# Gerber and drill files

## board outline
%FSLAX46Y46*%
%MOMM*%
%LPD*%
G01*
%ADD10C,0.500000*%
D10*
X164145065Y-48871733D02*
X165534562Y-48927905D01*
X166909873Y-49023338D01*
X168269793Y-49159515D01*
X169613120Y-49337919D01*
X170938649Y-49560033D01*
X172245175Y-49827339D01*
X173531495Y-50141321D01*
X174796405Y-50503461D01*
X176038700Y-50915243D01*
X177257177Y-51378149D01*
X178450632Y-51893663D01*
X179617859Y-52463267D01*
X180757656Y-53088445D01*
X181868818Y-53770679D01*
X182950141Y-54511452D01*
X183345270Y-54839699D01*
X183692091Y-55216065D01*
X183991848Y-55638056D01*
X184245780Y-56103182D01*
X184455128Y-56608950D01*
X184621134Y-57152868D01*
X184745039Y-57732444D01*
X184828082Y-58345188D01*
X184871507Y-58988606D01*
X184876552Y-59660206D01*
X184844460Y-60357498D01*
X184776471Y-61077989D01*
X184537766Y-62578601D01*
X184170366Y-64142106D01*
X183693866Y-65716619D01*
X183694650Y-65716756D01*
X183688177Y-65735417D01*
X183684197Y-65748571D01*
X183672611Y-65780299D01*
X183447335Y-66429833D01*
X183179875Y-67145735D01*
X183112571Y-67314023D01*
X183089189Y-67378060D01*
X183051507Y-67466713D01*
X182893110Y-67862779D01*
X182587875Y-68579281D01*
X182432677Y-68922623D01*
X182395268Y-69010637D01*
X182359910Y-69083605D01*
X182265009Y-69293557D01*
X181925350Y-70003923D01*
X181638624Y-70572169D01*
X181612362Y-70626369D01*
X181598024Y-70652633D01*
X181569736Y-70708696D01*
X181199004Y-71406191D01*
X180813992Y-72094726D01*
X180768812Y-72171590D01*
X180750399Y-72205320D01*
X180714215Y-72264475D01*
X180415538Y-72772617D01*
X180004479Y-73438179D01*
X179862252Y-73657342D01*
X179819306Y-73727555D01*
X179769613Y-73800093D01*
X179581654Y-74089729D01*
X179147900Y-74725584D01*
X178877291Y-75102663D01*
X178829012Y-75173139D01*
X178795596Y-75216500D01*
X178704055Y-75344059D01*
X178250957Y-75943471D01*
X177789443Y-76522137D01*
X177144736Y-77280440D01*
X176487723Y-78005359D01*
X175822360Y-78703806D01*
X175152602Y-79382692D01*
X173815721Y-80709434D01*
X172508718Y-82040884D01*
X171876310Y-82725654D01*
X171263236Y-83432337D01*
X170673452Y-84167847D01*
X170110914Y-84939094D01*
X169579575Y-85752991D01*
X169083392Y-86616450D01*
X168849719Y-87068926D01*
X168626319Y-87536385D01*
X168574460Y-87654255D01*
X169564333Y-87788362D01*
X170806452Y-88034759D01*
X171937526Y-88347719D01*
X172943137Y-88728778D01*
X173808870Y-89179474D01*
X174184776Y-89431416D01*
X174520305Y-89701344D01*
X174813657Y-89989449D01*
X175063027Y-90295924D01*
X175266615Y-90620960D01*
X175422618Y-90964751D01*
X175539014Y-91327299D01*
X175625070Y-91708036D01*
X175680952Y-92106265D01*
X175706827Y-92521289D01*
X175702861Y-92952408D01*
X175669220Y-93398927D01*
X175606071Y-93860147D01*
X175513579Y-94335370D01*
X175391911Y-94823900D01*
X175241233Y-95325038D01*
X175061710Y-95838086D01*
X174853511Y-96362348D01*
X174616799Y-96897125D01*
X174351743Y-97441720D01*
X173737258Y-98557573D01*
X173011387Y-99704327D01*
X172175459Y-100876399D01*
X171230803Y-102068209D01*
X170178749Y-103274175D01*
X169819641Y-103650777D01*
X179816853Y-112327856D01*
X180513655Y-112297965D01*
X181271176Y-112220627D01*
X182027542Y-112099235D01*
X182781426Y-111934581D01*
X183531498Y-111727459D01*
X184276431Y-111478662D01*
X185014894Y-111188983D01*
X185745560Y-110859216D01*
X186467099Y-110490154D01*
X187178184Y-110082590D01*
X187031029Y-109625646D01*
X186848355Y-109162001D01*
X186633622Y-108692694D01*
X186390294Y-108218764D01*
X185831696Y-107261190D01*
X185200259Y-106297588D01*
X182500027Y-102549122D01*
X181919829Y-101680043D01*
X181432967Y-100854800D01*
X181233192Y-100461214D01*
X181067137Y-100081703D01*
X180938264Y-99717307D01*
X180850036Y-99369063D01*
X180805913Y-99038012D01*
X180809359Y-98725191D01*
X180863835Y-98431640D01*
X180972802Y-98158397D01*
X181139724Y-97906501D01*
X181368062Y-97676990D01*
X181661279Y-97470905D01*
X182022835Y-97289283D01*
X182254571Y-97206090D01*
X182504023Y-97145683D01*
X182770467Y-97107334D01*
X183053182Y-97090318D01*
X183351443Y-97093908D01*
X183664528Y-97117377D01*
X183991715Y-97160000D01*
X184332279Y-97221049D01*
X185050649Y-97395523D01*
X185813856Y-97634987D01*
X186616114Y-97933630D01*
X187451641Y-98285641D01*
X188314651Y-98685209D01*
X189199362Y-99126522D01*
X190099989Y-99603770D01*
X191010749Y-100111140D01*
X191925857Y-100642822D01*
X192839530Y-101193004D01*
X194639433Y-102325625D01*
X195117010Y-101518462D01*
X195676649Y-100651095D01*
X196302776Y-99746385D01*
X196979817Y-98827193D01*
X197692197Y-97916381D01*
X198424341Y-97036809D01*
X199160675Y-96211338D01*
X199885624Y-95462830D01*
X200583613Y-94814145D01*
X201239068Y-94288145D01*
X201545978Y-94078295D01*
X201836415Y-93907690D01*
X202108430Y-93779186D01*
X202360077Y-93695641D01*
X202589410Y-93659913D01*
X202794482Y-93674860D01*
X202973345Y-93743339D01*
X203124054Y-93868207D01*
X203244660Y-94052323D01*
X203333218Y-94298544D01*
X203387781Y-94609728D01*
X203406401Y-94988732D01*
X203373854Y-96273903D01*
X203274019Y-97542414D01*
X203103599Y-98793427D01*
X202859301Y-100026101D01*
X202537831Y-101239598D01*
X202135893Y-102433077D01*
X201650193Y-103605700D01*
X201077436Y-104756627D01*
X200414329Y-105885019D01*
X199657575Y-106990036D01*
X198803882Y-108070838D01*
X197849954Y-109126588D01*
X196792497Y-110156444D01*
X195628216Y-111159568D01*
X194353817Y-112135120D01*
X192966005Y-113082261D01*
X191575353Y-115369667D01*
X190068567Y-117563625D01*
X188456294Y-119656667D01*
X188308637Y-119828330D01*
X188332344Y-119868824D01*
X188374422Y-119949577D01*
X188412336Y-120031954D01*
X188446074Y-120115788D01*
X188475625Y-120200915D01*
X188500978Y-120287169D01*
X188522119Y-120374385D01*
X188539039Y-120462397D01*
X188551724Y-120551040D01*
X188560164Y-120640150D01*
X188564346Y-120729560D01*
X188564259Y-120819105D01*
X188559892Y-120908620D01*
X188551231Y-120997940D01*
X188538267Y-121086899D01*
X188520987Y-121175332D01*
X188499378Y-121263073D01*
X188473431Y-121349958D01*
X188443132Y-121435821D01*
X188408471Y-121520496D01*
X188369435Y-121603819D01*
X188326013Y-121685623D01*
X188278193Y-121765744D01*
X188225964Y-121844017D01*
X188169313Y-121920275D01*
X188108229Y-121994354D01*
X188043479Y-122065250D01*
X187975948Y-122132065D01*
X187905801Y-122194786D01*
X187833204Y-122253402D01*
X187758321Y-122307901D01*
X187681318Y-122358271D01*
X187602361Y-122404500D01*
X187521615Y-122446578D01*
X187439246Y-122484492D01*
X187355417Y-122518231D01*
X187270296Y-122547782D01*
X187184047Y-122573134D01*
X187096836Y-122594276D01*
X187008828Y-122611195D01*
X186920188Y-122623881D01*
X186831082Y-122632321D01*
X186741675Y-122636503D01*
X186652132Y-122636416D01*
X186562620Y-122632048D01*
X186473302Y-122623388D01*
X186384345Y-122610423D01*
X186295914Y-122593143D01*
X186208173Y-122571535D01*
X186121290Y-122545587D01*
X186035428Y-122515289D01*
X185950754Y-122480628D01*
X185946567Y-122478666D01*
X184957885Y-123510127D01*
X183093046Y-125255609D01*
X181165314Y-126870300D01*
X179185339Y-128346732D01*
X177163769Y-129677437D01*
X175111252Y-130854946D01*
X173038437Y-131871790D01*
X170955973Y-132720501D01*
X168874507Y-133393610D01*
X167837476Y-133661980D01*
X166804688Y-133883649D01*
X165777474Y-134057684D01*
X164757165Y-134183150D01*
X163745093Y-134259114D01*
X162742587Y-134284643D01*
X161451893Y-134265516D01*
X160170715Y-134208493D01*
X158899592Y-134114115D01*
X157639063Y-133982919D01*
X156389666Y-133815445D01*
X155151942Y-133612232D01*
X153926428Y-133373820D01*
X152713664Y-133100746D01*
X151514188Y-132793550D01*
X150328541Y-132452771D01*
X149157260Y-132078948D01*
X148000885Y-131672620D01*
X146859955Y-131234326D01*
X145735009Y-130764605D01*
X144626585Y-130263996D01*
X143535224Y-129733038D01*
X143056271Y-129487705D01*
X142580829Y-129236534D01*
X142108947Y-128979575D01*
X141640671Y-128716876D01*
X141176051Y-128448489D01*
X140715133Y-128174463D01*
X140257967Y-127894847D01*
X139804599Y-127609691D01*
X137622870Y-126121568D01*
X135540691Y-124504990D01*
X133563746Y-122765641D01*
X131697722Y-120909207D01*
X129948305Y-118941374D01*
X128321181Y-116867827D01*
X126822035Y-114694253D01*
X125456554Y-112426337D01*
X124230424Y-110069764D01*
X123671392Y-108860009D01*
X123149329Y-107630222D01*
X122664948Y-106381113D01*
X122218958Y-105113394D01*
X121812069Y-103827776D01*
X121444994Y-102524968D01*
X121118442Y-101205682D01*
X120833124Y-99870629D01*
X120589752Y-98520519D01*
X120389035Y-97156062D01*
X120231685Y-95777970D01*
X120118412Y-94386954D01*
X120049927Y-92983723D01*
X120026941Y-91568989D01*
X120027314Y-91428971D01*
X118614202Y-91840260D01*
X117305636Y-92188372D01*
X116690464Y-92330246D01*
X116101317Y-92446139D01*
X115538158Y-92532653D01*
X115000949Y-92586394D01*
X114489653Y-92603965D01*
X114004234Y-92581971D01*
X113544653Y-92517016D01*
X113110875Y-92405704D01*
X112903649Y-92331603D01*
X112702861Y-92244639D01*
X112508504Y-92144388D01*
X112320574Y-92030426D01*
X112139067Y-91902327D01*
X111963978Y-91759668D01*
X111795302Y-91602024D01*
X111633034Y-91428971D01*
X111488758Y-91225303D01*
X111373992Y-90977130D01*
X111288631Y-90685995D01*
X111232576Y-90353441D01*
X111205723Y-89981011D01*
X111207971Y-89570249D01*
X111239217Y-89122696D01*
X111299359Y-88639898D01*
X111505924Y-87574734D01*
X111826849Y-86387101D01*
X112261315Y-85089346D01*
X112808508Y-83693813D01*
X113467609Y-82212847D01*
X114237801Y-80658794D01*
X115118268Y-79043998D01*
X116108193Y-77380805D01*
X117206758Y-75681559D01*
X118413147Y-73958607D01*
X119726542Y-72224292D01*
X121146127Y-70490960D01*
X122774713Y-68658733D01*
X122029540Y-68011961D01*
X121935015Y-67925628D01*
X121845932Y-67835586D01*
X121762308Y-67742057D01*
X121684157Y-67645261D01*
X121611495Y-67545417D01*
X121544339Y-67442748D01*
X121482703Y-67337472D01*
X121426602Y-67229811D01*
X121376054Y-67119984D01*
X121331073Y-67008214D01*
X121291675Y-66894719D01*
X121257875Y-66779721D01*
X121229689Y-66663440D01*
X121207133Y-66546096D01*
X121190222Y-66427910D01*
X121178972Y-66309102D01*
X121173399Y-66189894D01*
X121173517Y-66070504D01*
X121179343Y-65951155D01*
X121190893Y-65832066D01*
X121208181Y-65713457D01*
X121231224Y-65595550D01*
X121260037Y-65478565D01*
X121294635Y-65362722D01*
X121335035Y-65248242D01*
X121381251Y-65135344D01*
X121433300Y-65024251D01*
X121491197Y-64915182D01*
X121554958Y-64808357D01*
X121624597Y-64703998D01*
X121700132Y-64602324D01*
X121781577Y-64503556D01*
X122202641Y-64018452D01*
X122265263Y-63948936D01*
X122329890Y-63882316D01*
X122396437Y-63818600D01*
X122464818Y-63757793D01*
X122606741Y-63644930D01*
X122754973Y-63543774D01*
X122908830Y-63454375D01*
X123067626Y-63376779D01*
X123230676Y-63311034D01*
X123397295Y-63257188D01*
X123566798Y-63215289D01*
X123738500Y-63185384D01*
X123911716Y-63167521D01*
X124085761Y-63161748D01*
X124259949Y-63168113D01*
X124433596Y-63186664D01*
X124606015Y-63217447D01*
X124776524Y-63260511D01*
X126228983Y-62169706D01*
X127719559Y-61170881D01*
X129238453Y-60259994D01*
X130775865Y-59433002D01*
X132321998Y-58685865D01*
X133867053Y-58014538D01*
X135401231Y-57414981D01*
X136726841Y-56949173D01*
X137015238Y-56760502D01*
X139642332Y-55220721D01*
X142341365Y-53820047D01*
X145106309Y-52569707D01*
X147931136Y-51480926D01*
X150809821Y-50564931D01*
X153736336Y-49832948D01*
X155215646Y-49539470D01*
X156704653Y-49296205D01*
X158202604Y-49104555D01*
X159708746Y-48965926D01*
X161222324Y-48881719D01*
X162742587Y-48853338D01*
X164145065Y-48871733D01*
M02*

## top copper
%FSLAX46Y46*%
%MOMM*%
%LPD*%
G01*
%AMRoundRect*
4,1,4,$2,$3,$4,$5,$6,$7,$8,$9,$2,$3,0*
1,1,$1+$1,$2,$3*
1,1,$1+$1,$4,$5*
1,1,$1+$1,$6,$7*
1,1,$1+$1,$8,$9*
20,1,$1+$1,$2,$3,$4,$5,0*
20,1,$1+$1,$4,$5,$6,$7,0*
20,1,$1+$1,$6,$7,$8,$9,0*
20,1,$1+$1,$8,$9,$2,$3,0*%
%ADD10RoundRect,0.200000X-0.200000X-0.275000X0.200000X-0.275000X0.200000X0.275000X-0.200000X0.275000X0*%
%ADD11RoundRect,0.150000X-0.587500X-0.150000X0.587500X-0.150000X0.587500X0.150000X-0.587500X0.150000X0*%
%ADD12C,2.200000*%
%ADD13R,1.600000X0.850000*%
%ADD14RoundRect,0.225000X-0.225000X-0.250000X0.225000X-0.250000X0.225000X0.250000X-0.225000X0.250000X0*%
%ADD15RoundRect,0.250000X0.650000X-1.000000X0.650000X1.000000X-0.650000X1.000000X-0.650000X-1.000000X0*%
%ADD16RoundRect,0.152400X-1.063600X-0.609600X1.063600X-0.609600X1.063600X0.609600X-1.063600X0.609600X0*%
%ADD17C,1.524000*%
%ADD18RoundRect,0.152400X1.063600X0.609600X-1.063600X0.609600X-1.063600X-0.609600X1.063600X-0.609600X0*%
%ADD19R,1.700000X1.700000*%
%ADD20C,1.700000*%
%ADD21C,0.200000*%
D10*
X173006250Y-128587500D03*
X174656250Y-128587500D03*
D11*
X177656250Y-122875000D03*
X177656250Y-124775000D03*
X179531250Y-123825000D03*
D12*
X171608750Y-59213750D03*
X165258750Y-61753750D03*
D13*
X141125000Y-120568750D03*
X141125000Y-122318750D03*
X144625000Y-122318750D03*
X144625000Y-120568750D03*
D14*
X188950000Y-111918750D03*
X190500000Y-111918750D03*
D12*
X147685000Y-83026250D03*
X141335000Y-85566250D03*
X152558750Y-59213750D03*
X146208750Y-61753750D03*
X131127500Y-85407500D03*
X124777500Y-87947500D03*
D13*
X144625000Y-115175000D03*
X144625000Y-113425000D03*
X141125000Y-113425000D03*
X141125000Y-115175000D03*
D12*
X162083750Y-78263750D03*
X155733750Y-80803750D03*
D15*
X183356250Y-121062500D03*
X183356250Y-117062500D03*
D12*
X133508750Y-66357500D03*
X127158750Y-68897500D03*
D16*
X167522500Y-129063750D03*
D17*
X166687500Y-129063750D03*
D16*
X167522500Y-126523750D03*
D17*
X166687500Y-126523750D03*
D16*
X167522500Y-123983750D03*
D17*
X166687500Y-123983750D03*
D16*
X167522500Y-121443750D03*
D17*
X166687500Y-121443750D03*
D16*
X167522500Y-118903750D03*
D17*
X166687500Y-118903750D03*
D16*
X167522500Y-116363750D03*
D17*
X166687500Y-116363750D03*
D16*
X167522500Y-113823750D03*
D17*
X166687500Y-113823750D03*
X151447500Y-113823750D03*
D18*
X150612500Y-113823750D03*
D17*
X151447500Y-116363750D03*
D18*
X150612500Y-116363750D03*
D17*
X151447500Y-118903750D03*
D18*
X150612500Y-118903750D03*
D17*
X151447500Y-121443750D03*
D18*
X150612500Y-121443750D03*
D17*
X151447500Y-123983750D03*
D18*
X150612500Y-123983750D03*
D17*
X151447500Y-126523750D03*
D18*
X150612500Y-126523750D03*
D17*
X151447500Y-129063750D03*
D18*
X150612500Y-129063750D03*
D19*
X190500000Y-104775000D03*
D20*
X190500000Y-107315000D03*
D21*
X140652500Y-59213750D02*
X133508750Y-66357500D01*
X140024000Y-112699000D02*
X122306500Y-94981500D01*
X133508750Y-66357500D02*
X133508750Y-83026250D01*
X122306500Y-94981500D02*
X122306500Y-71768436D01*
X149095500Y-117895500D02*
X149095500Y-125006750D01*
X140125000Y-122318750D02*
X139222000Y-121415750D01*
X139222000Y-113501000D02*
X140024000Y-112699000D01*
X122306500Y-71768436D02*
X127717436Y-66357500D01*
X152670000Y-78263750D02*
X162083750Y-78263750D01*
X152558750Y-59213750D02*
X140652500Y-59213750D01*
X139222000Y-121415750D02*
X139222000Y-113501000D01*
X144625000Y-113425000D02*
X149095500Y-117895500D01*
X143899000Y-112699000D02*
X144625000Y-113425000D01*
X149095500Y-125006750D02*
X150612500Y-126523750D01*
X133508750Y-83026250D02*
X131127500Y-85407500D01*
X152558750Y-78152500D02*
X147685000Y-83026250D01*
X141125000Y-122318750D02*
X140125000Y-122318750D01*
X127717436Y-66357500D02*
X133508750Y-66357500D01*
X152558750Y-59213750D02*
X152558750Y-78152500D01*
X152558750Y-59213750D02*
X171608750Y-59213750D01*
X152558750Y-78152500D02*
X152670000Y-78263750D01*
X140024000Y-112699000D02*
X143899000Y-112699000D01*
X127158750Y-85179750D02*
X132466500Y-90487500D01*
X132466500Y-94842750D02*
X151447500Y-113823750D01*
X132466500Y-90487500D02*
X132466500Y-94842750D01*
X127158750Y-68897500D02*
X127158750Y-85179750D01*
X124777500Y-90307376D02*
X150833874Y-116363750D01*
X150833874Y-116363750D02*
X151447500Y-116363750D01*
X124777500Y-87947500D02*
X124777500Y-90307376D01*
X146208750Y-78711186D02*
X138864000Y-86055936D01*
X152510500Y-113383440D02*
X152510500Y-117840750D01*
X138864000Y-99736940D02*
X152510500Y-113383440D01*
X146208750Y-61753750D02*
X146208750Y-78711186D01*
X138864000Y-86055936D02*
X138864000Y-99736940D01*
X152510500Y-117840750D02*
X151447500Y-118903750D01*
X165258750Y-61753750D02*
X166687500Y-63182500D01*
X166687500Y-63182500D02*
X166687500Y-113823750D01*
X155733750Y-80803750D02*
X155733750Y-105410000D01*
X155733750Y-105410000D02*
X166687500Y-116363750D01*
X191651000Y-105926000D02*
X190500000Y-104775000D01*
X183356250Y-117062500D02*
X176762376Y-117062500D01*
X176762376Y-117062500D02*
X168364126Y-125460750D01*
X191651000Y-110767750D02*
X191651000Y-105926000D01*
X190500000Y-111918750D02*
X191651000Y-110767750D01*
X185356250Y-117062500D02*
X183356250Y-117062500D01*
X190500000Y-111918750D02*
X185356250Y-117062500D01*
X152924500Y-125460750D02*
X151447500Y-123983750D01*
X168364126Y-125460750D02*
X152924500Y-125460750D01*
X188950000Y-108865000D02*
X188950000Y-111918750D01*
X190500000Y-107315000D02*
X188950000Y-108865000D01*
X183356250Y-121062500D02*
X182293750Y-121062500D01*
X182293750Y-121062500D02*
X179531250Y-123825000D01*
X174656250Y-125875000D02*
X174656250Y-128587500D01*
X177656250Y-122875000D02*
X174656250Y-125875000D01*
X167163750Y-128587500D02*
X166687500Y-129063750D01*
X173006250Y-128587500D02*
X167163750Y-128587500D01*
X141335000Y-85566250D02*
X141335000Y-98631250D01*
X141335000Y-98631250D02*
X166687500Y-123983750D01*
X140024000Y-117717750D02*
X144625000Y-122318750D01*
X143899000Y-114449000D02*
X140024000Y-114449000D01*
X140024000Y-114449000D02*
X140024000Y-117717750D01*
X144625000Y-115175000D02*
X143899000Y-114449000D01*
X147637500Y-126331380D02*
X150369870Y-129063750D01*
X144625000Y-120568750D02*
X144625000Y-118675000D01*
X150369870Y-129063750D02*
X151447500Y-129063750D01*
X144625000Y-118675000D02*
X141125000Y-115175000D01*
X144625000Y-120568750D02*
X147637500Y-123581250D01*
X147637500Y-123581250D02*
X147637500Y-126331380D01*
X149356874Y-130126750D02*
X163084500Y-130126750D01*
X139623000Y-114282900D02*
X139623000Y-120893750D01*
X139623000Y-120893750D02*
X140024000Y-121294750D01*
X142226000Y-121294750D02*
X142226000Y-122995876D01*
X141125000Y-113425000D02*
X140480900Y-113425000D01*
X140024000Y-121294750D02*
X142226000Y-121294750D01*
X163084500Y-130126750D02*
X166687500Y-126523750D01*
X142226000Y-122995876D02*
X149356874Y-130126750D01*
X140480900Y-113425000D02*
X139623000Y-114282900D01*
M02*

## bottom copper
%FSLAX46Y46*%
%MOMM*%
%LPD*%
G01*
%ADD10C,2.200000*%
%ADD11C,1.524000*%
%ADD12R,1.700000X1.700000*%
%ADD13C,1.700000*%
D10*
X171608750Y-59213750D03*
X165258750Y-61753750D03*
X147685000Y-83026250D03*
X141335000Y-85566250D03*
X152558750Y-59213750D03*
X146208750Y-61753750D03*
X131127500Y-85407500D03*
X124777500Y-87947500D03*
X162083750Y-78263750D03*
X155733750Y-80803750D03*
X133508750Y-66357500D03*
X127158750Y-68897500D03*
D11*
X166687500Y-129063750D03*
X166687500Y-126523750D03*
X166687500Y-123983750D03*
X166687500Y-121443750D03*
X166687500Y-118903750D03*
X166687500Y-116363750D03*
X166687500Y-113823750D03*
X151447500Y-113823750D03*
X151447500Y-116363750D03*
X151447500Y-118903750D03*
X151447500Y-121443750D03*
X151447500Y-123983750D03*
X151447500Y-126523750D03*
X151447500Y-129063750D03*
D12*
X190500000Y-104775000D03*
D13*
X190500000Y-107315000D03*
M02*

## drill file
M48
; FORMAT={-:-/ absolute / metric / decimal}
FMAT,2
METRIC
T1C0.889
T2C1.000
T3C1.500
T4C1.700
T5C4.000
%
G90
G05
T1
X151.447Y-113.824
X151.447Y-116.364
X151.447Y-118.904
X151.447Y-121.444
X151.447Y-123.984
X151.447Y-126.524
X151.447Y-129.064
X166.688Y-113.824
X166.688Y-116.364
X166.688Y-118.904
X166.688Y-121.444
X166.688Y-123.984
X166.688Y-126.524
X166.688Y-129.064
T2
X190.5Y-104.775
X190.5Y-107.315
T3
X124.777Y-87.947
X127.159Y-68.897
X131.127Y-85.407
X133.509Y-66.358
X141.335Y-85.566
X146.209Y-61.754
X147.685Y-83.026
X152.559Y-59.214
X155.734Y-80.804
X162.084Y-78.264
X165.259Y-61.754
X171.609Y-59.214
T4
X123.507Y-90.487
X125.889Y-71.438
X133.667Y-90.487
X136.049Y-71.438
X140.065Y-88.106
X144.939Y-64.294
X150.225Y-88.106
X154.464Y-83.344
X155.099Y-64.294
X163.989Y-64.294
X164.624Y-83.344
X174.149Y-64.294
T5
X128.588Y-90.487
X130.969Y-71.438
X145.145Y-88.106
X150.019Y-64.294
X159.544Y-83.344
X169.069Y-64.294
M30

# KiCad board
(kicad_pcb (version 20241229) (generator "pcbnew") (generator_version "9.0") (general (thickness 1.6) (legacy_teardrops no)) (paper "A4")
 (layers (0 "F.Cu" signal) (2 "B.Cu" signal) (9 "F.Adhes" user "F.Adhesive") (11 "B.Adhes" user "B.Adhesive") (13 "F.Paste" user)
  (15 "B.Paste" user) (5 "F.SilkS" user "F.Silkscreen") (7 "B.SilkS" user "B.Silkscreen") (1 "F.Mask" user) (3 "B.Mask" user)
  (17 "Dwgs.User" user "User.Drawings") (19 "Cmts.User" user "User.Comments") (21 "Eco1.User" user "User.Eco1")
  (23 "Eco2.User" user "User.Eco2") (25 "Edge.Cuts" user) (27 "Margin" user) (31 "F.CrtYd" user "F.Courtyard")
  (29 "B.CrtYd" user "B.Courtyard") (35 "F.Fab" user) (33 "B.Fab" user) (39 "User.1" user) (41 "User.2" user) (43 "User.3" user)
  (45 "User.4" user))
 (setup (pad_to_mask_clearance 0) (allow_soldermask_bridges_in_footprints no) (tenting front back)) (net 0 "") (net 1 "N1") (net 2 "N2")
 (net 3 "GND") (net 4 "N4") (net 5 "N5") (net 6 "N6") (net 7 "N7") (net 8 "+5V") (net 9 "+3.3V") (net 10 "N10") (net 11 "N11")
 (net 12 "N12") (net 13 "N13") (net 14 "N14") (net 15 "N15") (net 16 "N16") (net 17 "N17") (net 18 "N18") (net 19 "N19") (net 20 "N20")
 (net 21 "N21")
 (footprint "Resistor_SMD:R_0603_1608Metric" (layer "F.Cu") (at 173.83125 128.5875)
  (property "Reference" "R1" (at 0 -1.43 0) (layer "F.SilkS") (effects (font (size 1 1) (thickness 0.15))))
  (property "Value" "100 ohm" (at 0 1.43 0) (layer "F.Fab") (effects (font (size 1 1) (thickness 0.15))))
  (pad "1" smd roundrect (at -0.825 0) (size 0.8 0.95) (layers "F.Cu" "F.Mask" "F.Paste") (roundrect_rratio 0.25) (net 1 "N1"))
  (pad "2" smd roundrect (at 0.825 0) (size 0.8 0.95) (layers "F.Cu" "F.Mask" "F.Paste") (roundrect_rratio 0.25) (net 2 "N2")))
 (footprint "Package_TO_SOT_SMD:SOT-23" (layer "F.Cu") (at 178.59375 123.825)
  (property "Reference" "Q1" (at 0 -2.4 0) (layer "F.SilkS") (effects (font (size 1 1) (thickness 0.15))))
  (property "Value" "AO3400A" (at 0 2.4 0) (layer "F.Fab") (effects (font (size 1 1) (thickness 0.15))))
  (pad "1" smd roundrect (at -0.9375 -0.95) (size 1.475 0.6) (layers "F.Cu" "F.Mask" "F.Paste") (roundrect_rratio 0.25) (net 2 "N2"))
  (pad "2" smd roundrect (at -0.9375 0.95) (size 1.475 0.6) (layers "F.Cu" "F.Mask" "F.Paste") (roundrect_rratio 0.25) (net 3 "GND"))
  (pad "3" smd roundrect (at 0.9375 0) (size 1.475 0.6) (layers "F.Cu" "F.Mask" "F.Paste") (roundrect_rratio 0.25) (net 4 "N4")))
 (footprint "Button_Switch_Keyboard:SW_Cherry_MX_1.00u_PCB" (layer "F.Cu") (at 171.60875 59.21375)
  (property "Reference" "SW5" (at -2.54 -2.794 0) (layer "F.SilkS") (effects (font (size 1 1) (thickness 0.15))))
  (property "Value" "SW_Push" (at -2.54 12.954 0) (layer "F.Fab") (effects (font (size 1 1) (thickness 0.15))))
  (pad "" np_thru_hole circle (at -7.62 5.08) (size 1.7 1.7) (drill 1.7) (layers "*.Cu" "*.Mask"))
  (pad "" np_thru_hole circle (at -2.54 5.08) (size 4 4) (drill 4) (layers "*.Cu" "*.Mask"))
  (pad "" np_thru_hole circle (at 2.54 5.08) (size 1.7 1.7) (drill 1.7) (layers "*.Cu" "*.Mask"))
  (pad "1" thru_hole circle (at 0 0) (size 2.2 2.2) (drill 1.5) (layers "*.Cu" "*.Mask") (remove_unused_layers no) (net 3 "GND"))
  (pad "2" thru_hole circle (at -6.35 2.54) (size 2.2 2.2) (drill 1.5) (layers "*.Cu" "*.Mask") (remove_unused_layers no) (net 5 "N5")))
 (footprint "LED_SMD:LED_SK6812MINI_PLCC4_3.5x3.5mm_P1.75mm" (layer "F.Cu") (at 142.875 121.44375)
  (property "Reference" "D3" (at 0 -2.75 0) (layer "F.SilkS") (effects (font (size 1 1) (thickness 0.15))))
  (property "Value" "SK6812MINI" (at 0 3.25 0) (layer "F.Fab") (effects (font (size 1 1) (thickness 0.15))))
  (pad "1" smd rect (at -1.75 -0.875) (size 1.6 0.85) (layers "F.Cu" "F.Mask" "F.Paste") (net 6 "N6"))
  (pad "2" smd rect (at -1.75 0.875) (size 1.6 0.85) (layers "F.Cu" "F.Mask" "F.Paste") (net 3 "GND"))
  (pad "3" smd rect (at 1.75 0.875) (size 1.6 0.85) (layers "F.Cu" "F.Mask" "F.Paste") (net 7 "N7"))
  (pad "4" smd rect (at 1.75 -0.875) (size 1.6 0.85) (layers "F.Cu" "F.Mask" "F.Paste") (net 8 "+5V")))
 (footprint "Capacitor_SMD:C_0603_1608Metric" (layer "F.Cu") (at 189.725 111.91875)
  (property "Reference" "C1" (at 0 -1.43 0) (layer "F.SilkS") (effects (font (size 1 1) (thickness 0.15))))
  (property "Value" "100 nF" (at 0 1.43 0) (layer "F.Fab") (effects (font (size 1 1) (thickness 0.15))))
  (pad "1" smd roundrect (at -0.775 0) (size 0.9 0.95) (layers "F.Cu" "F.Mask" "F.Paste") (roundrect_rratio 0.25) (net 4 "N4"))
  (pad "2" smd roundrect (at 0.775 0) (size 0.9 0.95) (layers "F.Cu" "F.Mask" "F.Paste") (roundrect_rratio 0.25) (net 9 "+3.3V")))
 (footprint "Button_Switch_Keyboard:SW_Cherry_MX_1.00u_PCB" (layer "F.Cu") (at 147.685 83.02625)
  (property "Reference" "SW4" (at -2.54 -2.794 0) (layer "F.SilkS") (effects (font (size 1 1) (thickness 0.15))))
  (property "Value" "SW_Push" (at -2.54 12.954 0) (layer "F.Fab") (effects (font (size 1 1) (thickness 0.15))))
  (pad "" np_thru_hole circle (at -7.62 5.08) (size 1.7 1.7) (drill 1.7) (layers "*.Cu" "*.Mask"))
  (pad "" np_thru_hole circle (at -2.54 5.08) (size 4 4) (drill 4) (layers "*.Cu" "*.Mask"))
  (pad "" np_thru_hole circle (at 2.54 5.08) (size 1.7 1.7) (drill 1.7) (layers "*.Cu" "*.Mask"))
  (pad "1" thru_hole circle (at 0 0) (size 2.2 2.2) (drill 1.5) (layers "*.Cu" "*.Mask") (remove_unused_layers no) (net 3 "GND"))
  (pad "2" thru_hole circle (at -6.35 2.54) (size 2.2 2.2) (drill 1.5) (layers "*.Cu" "*.Mask") (remove_unused_layers no) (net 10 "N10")))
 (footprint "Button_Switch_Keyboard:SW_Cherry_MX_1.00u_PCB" (layer "F.Cu") (at 152.55875 59.21375)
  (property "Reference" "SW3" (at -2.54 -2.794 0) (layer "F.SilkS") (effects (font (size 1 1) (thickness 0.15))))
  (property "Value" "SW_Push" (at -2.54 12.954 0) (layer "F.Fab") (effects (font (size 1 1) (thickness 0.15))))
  (pad "" np_thru_hole circle (at -7.62 5.08) (size 1.7 1.7) (drill 1.7) (layers "*.Cu" "*.Mask"))
  (pad "" np_thru_hole circle (at -2.54 5.08) (size 4 4) (drill 4) (layers "*.Cu" "*.Mask"))
  (pad "" np_thru_hole circle (at 2.54 5.08) (size 1.7 1.7) (drill 1.7) (layers "*.Cu" "*.Mask"))
  (pad "1" thru_hole circle (at 0 0) (size 2.2 2.2) (drill 1.5) (layers "*.Cu" "*.Mask") (remove_unused_layers no) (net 3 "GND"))
  (pad "2" thru_hole circle (at -6.35 2.54) (size 2.2 2.2) (drill 1.5) (layers "*.Cu" "*.Mask") (remove_unused_layers no) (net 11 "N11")))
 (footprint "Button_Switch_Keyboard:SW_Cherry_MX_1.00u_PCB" (layer "F.Cu") (at 131.1275 85.4075)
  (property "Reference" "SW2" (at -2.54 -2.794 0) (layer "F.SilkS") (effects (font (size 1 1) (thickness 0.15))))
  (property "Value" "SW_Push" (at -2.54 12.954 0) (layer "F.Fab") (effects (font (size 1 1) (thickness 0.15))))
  (pad "" np_thru_hole circle (at -7.62 5.08) (size 1.7 1.7) (drill 1.7) (layers "*.Cu" "*.Mask"))
  (pad "" np_thru_hole circle (at -2.54 5.08) (size 4 4) (drill 4) (layers "*.Cu" "*.Mask"))
  (pad "" np_thru_hole circle (at 2.54 5.08) (size 1.7 1.7) (drill 1.7) (layers "*.Cu" "*.Mask"))
  (pad "1" thru_hole circle (at 0 0) (size 2.2 2.2) (drill 1.5) (layers "*.Cu" "*.Mask") (remove_unused_layers no) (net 3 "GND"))
  (pad "2" thru_hole circle (at -6.35 2.54) (size 2.2 2.2) (drill 1.5) (layers "*.Cu" "*.Mask") (remove_unused_layers no) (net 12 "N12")))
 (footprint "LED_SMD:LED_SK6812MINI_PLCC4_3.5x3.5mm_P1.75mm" (layer "F.Cu") (at 142.875 114.3 180)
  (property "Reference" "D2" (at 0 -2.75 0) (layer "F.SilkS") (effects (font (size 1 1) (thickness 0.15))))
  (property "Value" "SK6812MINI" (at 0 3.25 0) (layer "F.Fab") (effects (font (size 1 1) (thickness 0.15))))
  (pad "1" smd rect (at -1.75 -0.875 180) (size 1.6 0.85) (layers "F.Cu" "F.Mask" "F.Paste") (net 7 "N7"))
  (pad "2" smd rect (at -1.75 0.875 180) (size 1.6 0.85) (layers "F.Cu" "F.Mask" "F.Paste") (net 3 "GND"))
  (pad "3" smd rect (at 1.75 0.875 180) (size 1.6 0.85) (layers "F.Cu" "F.Mask" "F.Paste") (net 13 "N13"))
  (pad "4" smd rect (at 1.75 -0.875 180) (size 1.6 0.85) (layers "F.Cu" "F.Mask" "F.Paste") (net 8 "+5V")))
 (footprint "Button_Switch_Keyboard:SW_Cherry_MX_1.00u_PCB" (layer "F.Cu") (at 162.08375 78.26375)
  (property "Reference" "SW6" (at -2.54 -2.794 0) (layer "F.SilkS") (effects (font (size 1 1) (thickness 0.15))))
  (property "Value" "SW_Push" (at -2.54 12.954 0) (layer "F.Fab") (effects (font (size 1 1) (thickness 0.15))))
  (pad "" np_thru_hole circle (at -7.62 5.08) (size 1.7 1.7) (drill 1.7) (layers "*.Cu" "*.Mask"))
  (pad "" np_thru_hole circle (at -2.54 5.08) (size 4 4) (drill 4) (layers "*.Cu" "*.Mask"))
  (pad "" np_thru_hole circle (at 2.54 5.08) (size 1.7 1.7) (drill 1.7) (layers "*.Cu" "*.Mask"))
  (pad "1" thru_hole circle (at 0 0) (size 2.2 2.2) (drill 1.5) (layers "*.Cu" "*.Mask") (remove_unused_layers no) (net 3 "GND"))
  (pad "2" thru_hole circle (at -6.35 2.54) (size 2.2 2.2) (drill 1.5) (layers "*.Cu" "*.Mask") (remove_unused_layers no) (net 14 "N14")))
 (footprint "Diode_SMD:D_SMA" (layer "F.Cu") (at 183.35625 119.0625 90)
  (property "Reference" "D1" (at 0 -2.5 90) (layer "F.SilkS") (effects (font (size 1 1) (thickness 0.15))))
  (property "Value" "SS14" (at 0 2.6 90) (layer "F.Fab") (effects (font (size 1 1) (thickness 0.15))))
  (pad "1" smd roundrect (at -2 0 90) (size 2.5 1.8) (layers "F.Cu" "F.Mask" "F.Paste") (roundrect_rratio 0.1388888889) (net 4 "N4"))
  (pad "2" smd roundrect (at 2 0 90) (size 2.5 1.8) (layers "F.Cu" "F.Mask" "F.Paste") (roundrect_rratio 0.1388888889) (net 9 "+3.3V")))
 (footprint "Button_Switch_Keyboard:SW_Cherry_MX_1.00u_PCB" (layer "F.Cu") (at 133.50875 66.3575)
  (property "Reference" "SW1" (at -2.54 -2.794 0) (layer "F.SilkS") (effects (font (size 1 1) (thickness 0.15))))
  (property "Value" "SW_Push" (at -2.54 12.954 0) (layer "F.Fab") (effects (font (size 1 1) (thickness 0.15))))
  (pad "" np_thru_hole circle (at -7.62 5.08) (size 1.7 1.7) (drill 1.7) (layers "*.Cu" "*.Mask"))
  (pad "" np_thru_hole circle (at -2.54 5.08) (size 4 4) (drill 4) (layers "*.Cu" "*.Mask"))
  (pad "" np_thru_hole circle (at 2.54 5.08) (size 1.7 1.7) (drill 1.7) (layers "*.Cu" "*.Mask"))
  (pad "1" thru_hole circle (at 0 0) (size 2.2 2.2) (drill 1.5) (layers "*.Cu" "*.Mask") (remove_unused_layers no) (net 3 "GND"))
  (pad "2" thru_hole circle (at -6.35 2.54) (size 2.2 2.2) (drill 1.5) (layers "*.Cu" "*.Mask") (remove_unused_layers no) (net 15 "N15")))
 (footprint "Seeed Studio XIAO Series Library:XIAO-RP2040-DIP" (layer "F.Cu") (at 159.0675 121.44375 180)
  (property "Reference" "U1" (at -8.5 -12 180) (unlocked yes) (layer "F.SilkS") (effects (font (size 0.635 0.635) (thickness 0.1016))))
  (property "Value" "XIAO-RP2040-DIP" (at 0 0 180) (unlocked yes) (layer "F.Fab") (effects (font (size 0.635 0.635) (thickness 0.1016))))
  (pad "1" smd roundrect (at -8.455 -7.62) (size 2.432 1.524) (layers "F.Cu" "F.Mask") (roundrect_rratio 0.1) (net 1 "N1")
   (thermal_bridge_angle 45))
  (pad "1" thru_hole circle (at -7.62 -7.62) (size 1.524 1.524) (drill 0.889) (layers "*.Cu" "*.Mask") (remove_unused_layers no)
   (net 1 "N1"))
  (pad "2" smd roundrect (at -8.455 -5.08) (size 2.432 1.524) (layers "F.Cu" "F.Mask") (roundrect_rratio 0.1) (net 13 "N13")
   (thermal_bridge_angle 45))
  (pad "2" thru_hole circle (at -7.62 -5.08) (size 1.524 1.524) (drill 0.889) (layers "*.Cu" "*.Mask") (remove_unused_layers no)
   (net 13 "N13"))
  (pad "3" smd roundrect (at -8.455 -2.54) (size 2.432 1.524) (layers "F.Cu" "F.Mask") (roundrect_rratio 0.1) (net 10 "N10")
   (thermal_bridge_angle 45))
  (pad "3" thru_hole circle (at -7.62 -2.54) (size 1.524 1.524) (drill 0.889) (layers "*.Cu" "*.Mask") (remove_unused_layers no)
   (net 10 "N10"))
  (pad "4" smd roundrect (at -8.455 0) (size 2.432 1.524) (layers "F.Cu" "F.Mask") (roundrect_rratio 0.1) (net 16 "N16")
   (thermal_bridge_angle 45))
  (pad "4" thru_hole circle (at -7.62 0) (size 1.524 1.524) (drill 0.889) (layers "*.Cu" "*.Mask") (remove_unused_layers no) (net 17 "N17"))
  (pad "5" smd roundrect (at -8.455 2.54) (size 2.432 1.524) (layers "F.Cu" "F.Mask") (roundrect_rratio 0.1) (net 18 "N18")
   (thermal_bridge_angle 45))
  (pad "5" thru_hole circle (at -7.62 2.54) (size 1.524 1.524) (drill 0.889) (layers "*.Cu" "*.Mask") (remove_unused_layers no)
   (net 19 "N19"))
  (pad "6" smd roundrect (at -8.455 5.08) (size 2.432 1.524) (layers "F.Cu" "F.Mask") (roundrect_rratio 0.1) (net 14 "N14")
   (thermal_bridge_angle 45))
  (pad "6" thru_hole circle (at -7.62 5.08) (size 1.524 1.524) (drill 0.889) (layers "*.Cu" "*.Mask") (remove_unused_layers no)
   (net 14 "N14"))
  (pad "7" smd roundrect (at -8.455 7.62) (size 2.432 1.524) (layers "F.Cu" "F.Mask") (roundrect_rratio 0.1) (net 5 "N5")
   (thermal_bridge_angle 45))
  (pad "7" thru_hole circle (at -7.62 7.62) (size 1.524 1.524) (drill 0.889) (layers "*.Cu" "*.Mask") (remove_unused_layers no) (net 5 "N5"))
  (pad "8" thru_hole circle (at 7.62 7.62 180) (size 1.524 1.524) (drill 0.889) (layers "*.Cu" "*.Mask") (remove_unused_layers no)
   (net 15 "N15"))
  (pad "8" smd roundrect (at 8.455 7.62 180) (size 2.432 1.524) (layers "F.Cu" "F.Mask") (roundrect_rratio 0.1) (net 15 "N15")
   (thermal_bridge_angle 45))
  (pad "9" thru_hole circle (at 7.62 5.08 180) (size 1.524 1.524) (drill 0.889) (layers "*.Cu" "*.Mask") (remove_unused_layers no)
   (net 12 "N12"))
  (pad "9" smd roundrect (at 8.455 5.08 180) (size 2.432 1.524) (layers "F.Cu" "F.Mask") (roundrect_rratio 0.1) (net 12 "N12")
   (thermal_bridge_angle 45))
  (pad "10" thru_hole circle (at 7.62 2.54 180) (size 1.524 1.524) (drill 0.889) (layers "*.Cu" "*.Mask") (remove_unused_layers no)
   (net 11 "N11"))
  (pad "10" smd roundrect (at 8.455 2.54 180) (size 2.432 1.524) (layers "F.Cu" "F.Mask") (roundrect_rratio 0.1) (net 11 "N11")
   (thermal_bridge_angle 45))
  (pad "11" thru_hole circle (at 7.62 0 180) (size 1.524 1.524) (drill 0.889) (layers "*.Cu" "*.Mask") (remove_unused_layers no)
   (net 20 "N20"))
  (pad "11" smd roundrect (at 8.455 0 180) (size 2.432 1.524) (layers "F.Cu" "F.Mask") (roundrect_rratio 0.1) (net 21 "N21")
   (thermal_bridge_angle 45))
  (pad "12" thru_hole circle (at 7.62 -2.54 180) (size 1.524 1.524) (drill 0.889) (layers "*.Cu" "*.Mask") (remove_unused_layers no)
   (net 9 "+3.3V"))
  (pad "12" smd roundrect (at 8.455 -2.54 180) (size 2.432 1.524) (layers "F.Cu" "F.Mask") (roundrect_rratio 0.1) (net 9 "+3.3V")
   (thermal_bridge_angle 45))
  (pad "13" thru_hole circle (at 7.62 -5.08 180) (size 1.524 1.524) (drill 0.889) (layers "*.Cu" "*.Mask") (remove_unused_layers no)
   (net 3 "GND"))
  (pad "13" smd roundrect (at 8.455 -5.08 180) (size 2.432 1.524) (layers "F.Cu" "F.Mask") (roundrect_rratio 0.1) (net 3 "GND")
   (thermal_bridge_angle 45))
  (pad "14" thru_hole circle (at 7.62 -7.62 180) (size 1.524 1.524) (drill 0.889) (layers "*.Cu" "*.Mask") (remove_unused_layers no)
   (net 8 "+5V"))
  (pad "14" smd roundrect (at 8.455 -7.62 180) (size 2.432 1.524) (layers "F.Cu" "F.Mask") (roundrect_rratio 0.1) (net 8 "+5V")
   (thermal_bridge_angle 45)))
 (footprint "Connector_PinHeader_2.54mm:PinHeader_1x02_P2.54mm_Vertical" (layer "F.Cu") (at 190.5 104.775)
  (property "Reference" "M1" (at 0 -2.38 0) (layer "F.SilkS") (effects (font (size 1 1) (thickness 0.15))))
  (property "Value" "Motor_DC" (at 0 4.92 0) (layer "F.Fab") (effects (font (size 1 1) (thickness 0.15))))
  (pad "1" thru_hole rect (at 0 0) (size 1.7 1.7) (drill 1) (layers "*.Cu" "*.Mask") (remove_unused_layers no) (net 9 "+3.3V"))
  (pad "2" thru_hole circle (at 0 2.54) (size 1.7 1.7) (drill 1) (layers "*.Cu" "*.Mask") (remove_unused_layers no) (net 4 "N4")))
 (gr_poly
  (pts (xy 164.145065 48.871733) (xy 165.534562 48.927905) (xy 166.909873 49.023338) (xy 168.269793 49.159515) (xy 169.61312 49.337919)
   (xy 170.938649 49.560033) (xy 172.245175 49.827339) (xy 173.531495 50.141321) (xy 174.796405 50.503461) (xy 176.0387 50.915243)
   (xy 177.257177 51.378149) (xy 178.450632 51.893663) (xy 179.617859 52.463267) (xy 180.757656 53.088445) (xy 181.868818 53.770679)
   (xy 182.950141 54.511452) (xy 183.34527 54.839699) (xy 183.692091 55.216065) (xy 183.991848 55.638056) (xy 184.24578 56.103182)
   (xy 184.455128 56.60895) (xy 184.621134 57.152868) (xy 184.745039 57.732444) (xy 184.828082 58.345188) (xy 184.871507 58.988606)
   (xy 184.876552 59.660206) (xy 184.84446 60.357498) (xy 184.776471 61.077989) (xy 184.537766 62.578601) (xy 184.170366 64.142106)
   (xy 183.693866 65.716619) (xy 183.69465 65.716756) (xy 183.688177 65.735417) (xy 183.684197 65.748571) (xy 183.672611 65.780299)
   (xy 183.447335 66.429833) (xy 183.179875 67.145735) (xy 183.112571 67.314023) (xy 183.089189 67.37806) (xy 183.051507 67.466713)
   (xy 182.89311 67.862779) (xy 182.587875 68.579281) (xy 182.432677 68.922623) (xy 182.395268 69.010637) (xy 182.35991 69.083605)
   (xy 182.265009 69.293557) (xy 181.92535 70.003923) (xy 181.638624 70.572169) (xy 181.612362 70.626369) (xy 181.598024 70.652633)
   (xy 181.569736 70.708696) (xy 181.199004 71.406191) (xy 180.813992 72.094726) (xy 180.768812 72.17159) (xy 180.750399 72.20532)
   (xy 180.714215 72.264475) (xy 180.415538 72.772617) (xy 180.004479 73.438179) (xy 179.862252 73.657342) (xy 179.819306 73.727555)
   (xy 179.769613 73.800093) (xy 179.581654 74.089729) (xy 179.1479 74.725584) (xy 178.877291 75.102663) (xy 178.829012 75.173139)
   (xy 178.795596 75.2165) (xy 178.704055 75.344059) (xy 178.250957 75.943471) (xy 177.789443 76.522137) (xy 177.144736 77.28044)
   (xy 176.487723 78.005359) (xy 175.82236 78.703806) (xy 175.152602 79.382692) (xy 173.815721 80.709434) (xy 172.508718 82.040884)
   (xy 171.87631 82.725654) (xy 171.263236 83.432337) (xy 170.673452 84.167847) (xy 170.110914 84.939094) (xy 169.579575 85.752991)
   (xy 169.083392 86.61645) (xy 168.849719 87.068926) (xy 168.626319 87.536385) (xy 168.57446 87.654255) (xy 169.564333 87.788362)
   (xy 170.806452 88.034759) (xy 171.937526 88.347719) (xy 172.943137 88.728778) (xy 173.80887 89.179474) (xy 174.184776 89.431416)
   (xy 174.520305 89.701344) (xy 174.813657 89.989449) (xy 175.063027 90.295924) (xy 175.266615 90.62096) (xy 175.422618 90.964751)
   (xy 175.539014 91.327299) (xy 175.62507 91.708036) (xy 175.680952 92.106265) (xy 175.706827 92.521289) (xy 175.702861 92.952408)
   (xy 175.66922 93.398927) (xy 175.606071 93.860147) (xy 175.513579 94.33537) (xy 175.391911 94.8239) (xy 175.241233 95.325038)
   (xy 175.06171 95.838086) (xy 174.853511 96.362348) (xy 174.616799 96.897125) (xy 174.351743 97.44172) (xy 173.737258 98.557573)
   (xy 173.011387 99.704327) (xy 172.175459 100.876399) (xy 171.230803 102.068209) (xy 170.178749 103.274175) (xy 169.819641 103.650777)
   (xy 179.816853 112.327856) (xy 180.513655 112.297965) (xy 181.271176 112.220627) (xy 182.027542 112.099235) (xy 182.781426 111.934581)
   (xy 183.531498 111.727459) (xy 184.276431 111.478662) (xy 185.014894 111.188983) (xy 185.74556 110.859216) (xy 186.467099 110.490154)
   (xy 187.178184 110.08259) (xy 187.031029 109.625646) (xy 186.848355 109.162001) (xy 186.633622 108.692694) (xy 186.390294 108.218764)
   (xy 185.831696 107.26119) (xy 185.200259 106.297588) (xy 182.500027 102.549122) (xy 181.919829 101.680043) (xy 181.432967 100.8548)
   (xy 181.233192 100.461214) (xy 181.067137 100.081703) (xy 180.938264 99.717307) (xy 180.850036 99.369063) (xy 180.805913 99.038012)
   (xy 180.809359 98.725191) (xy 180.863835 98.43164) (xy 180.972802 98.158397) (xy 181.139724 97.906501) (xy 181.368062 97.67699)
   (xy 181.661279 97.470905) (xy 182.022835 97.289283) (xy 182.254571 97.20609) (xy 182.504023 97.145683) (xy 182.770467 97.107334)
   (xy 183.053182 97.090318) (xy 183.351443 97.093908) (xy 183.664528 97.117377) (xy 183.991715 97.16) (xy 184.332279 97.221049)
   (xy 185.050649 97.395523) (xy 185.813856 97.634987) (xy 186.616114 97.93363) (xy 187.451641 98.285641) (xy 188.314651 98.685209)
   (xy 189.199362 99.126522) (xy 190.099989 99.60377) (xy 191.010749 100.11114) (xy 191.925857 100.642822) (xy 192.83953 101.193004)
   (xy 194.639433 102.325625) (xy 195.11701 101.518462) (xy 195.676649 100.651095) (xy 196.302776 99.746385) (xy 196.979817 98.827193)
   (xy 197.692197 97.916381) (xy 198.424341 97.036809) (xy 199.160675 96.211338) (xy 199.885624 95.46283) (xy 200.583613 94.814145)
   (xy 201.239068 94.288145) (xy 201.545978 94.078295) (xy 201.836415 93.90769) (xy 202.10843 93.779186) (xy 202.360077 93.695641)
   (xy 202.58941 93.659913) (xy 202.794482 93.67486) (xy 202.973345 93.743339) (xy 203.124054 93.868207) (xy 203.24466 94.052323)
   (xy 203.333218 94.298544) (xy 203.387781 94.609728) (xy 203.406401 94.988732) (xy 203.373854 96.273903) (xy 203.274019 97.542414)
   (xy 203.103599 98.793427) (xy 202.859301 100.026101) (xy 202.537831 101.239598) (xy 202.135893 102.433077) (xy 201.650193 103.6057)
   (xy 201.077436 104.756627) (xy 200.414329 105.885019) (xy 199.657575 106.990036) (xy 198.803882 108.070838) (xy 197.849954 109.126588)
   (xy 196.792497 110.156444) (xy 195.628216 111.159568) (xy 194.353817 112.13512) (xy 192.966005 113.082261) (xy 191.575353 115.369667)
   (xy 190.068567 117.563625) (xy 188.456294 119.656667) (xy 188.308637 119.82833) (xy 188.332344 119.868824) (xy 188.374422 119.949577)
   (xy 188.412336 120.031954) (xy 188.446074 120.115788) (xy 188.475625 120.200915) (xy 188.500978 120.287169) (xy 188.522119 120.374385)
   (xy 188.539039 120.462397) (xy 188.551724 120.55104) (xy 188.560164 120.64015) (xy 188.564346 120.72956) (xy 188.564259 120.819105)
   (xy 188.559892 120.90862) (xy 188.551231 120.99794) (xy 188.538267 121.086899) (xy 188.520987 121.175332) (xy 188.499378 121.263073)
   (xy 188.473431 121.349958) (xy 188.443132 121.435821) (xy 188.408471 121.520496) (xy 188.369435 121.603819) (xy 188.326013 121.685623)
   (xy 188.278193 121.765744) (xy 188.225964 121.844017) (xy 188.169313 121.920275) (xy 188.108229 121.994354) (xy 188.043479 122.06525)
   (xy 187.975948 122.132065) (xy 187.905801 122.194786) (xy 187.833204 122.253402) (xy 187.758321 122.307901) (xy 187.681318 122.358271)
   (xy 187.602361 122.4045) (xy 187.521615 122.446578) (xy 187.439246 122.484492) (xy 187.355417 122.518231) (xy 187.270296 122.547782)
   (xy 187.184047 122.573134) (xy 187.096836 122.594276) (xy 187.008828 122.611195) (xy 186.920188 122.623881) (xy 186.831082 122.632321)
   (xy 186.741675 122.636503) (xy 186.652132 122.636416) (xy 186.56262 122.632048) (xy 186.473302 122.623388) (xy 186.384345 122.610423)
   (xy 186.295914 122.593143) (xy 186.208173 122.571535) (xy 186.12129 122.545587) (xy 186.035428 122.515289) (xy 185.950754 122.480628)
   (xy 185.946567 122.478666) (xy 184.957885 123.510127) (xy 183.093046 125.255609) (xy 181.165314 126.8703) (xy 179.185339 128.346732)
   (xy 177.163769 129.677437) (xy 175.111252 130.854946) (xy 173.038437 131.87179) (xy 170.955973 132.720501) (xy 168.874507 133.39361)
   (xy 167.837476 133.66198) (xy 166.804688 133.883649) (xy 165.777474 134.057684) (xy 164.757165 134.18315) (xy 163.745093 134.259114)
   (xy 162.742587 134.284643) (xy 161.451893 134.265516) (xy 160.170715 134.208493) (xy 158.899592 134.114115) (xy 157.639063 133.982919)
   (xy 156.389666 133.815445) (xy 155.151942 133.612232) (xy 153.926428 133.37382) (xy 152.713664 133.100746) (xy 151.514188 132.79355)
   (xy 150.328541 132.452771) (xy 149.15726 132.078948) (xy 148.000885 131.67262) (xy 146.859955 131.234326) (xy 145.735009 130.764605)
   (xy 144.626585 130.263996) (xy 143.535224 129.733038) (xy 143.056271 129.487705) (xy 142.580829 129.236534) (xy 142.108947 128.979575)
   (xy 141.640671 128.716876) (xy 141.176051 128.448489) (xy 140.715133 128.174463) (xy 140.257967 127.894847) (xy 139.804599 127.609691)
   (xy 137.62287 126.121568) (xy 135.540691 124.50499) (xy 133.563746 122.765641) (xy 131.697722 120.909207) (xy 129.948305 118.941374)
   (xy 128.321181 116.867827) (xy 126.822035 114.694253) (xy 125.456554 112.426337) (xy 124.230424 110.069764) (xy 123.671392 108.860009)
   (xy 123.149329 107.630222) (xy 122.664948 106.381113) (xy 122.218958 105.113394) (xy 121.812069 103.827776) (xy 121.444994 102.524968)
   (xy 121.118442 101.205682) (xy 120.833124 99.870629) (xy 120.589752 98.520519) (xy 120.389035 97.156062) (xy 120.231685 95.77797)
   (xy 120.118412 94.386954) (xy 120.049927 92.983723) (xy 120.026941 91.568989) (xy 120.027314 91.428971) (xy 118.614202 91.84026)
   (xy 117.305636 92.188372) (xy 116.690464 92.330246) (xy 116.101317 92.446139) (xy 115.538158 92.532653) (xy 115.000949 92.586394)
   (xy 114.489653 92.603965) (xy 114.004234 92.581971) (xy 113.544653 92.517016) (xy 113.110875 92.405704) (xy 112.903649 92.331603)
   (xy 112.702861 92.244639) (xy 112.508504 92.144388) (xy 112.320574 92.030426) (xy 112.139067 91.902327) (xy 111.963978 91.759668)
   (xy 111.795302 91.602024) (xy 111.633034 91.428971) (xy 111.488758 91.225303) (xy 111.373992 90.97713) (xy 111.288631 90.685995)
   (xy 111.232576 90.353441) (xy 111.205723 89.981011) (xy 111.207971 89.570249) (xy 111.239217 89.122696) (xy 111.299359 88.639898)
   (xy 111.505924 87.574734) (xy 111.826849 86.387101) (xy 112.261315 85.089346) (xy 112.808508 83.693813) (xy 113.467609 82.212847)
   (xy 114.237801 80.658794) (xy 115.118268 79.043998) (xy 116.108193 77.380805) (xy 117.206758 75.681559) (xy 118.413147 73.958607)
   (xy 119.726542 72.224292) (xy 121.146127 70.49096) (xy 122.774713 68.658733) (xy 122.02954 68.011961) (xy 121.935015 67.925628)
   (xy 121.845932 67.835586) (xy 121.762308 67.742057) (xy 121.684157 67.645261) (xy 121.611495 67.545417) (xy 121.544339 67.442748)
   (xy 121.482703 67.337472) (xy 121.426602 67.229811) (xy 121.376054 67.119984) (xy 121.331073 67.008214) (xy 121.291675 66.894719)
   (xy 121.257875 66.779721) (xy 121.229689 66.66344) (xy 121.207133 66.546096) (xy 121.190222 66.42791) (xy 121.178972 66.309102)
   (xy 121.173399 66.189894) (xy 121.173517 66.070504) (xy 121.179343 65.951155) (xy 121.190893 65.832066) (xy 121.208181 65.713457)
   (xy 121.231224 65.59555) (xy 121.260037 65.478565) (xy 121.294635 65.362722) (xy 121.335035 65.248242) (xy 121.381251 65.135344)
   (xy 121.4333 65.024251) (xy 121.491197 64.915182) (xy 121.554958 64.808357) (xy 121.624597 64.703998) (xy 121.700132 64.602324)
   (xy 121.781577 64.503556) (xy 122.202641 64.018452) (xy 122.265263 63.948936) (xy 122.32989 63.882316) (xy 122.396437 63.8186)
   (xy 122.464818 63.757793) (xy 122.606741 63.64493) (xy 122.754973 63.543774) (xy 122.90883 63.454375) (xy 123.067626 63.376779)
   (xy 123.230676 63.311034) (xy 123.397295 63.257188) (xy 123.566798 63.215289) (xy 123.7385 63.185384) (xy 123.911716 63.167521)
   (xy 124.085761 63.161748) (xy 124.259949 63.168113) (xy 124.433596 63.186664) (xy 124.606015 63.217447) (xy 124.776524 63.260511)
   (xy 126.228983 62.169706) (xy 127.719559 61.170881) (xy 129.238453 60.259994) (xy 130.775865 59.433002) (xy 132.321998 58.685865)
   (xy 133.867053 58.014538) (xy 135.401231 57.414981) (xy 136.726841 56.949173) (xy 137.015238 56.760502) (xy 139.642332 55.220721)
   (xy 142.341365 53.820047) (xy 145.106309 52.569707) (xy 147.931136 51.480926) (xy 150.809821 50.564931) (xy 153.736336 49.832948)
   (xy 155.215646 49.53947) (xy 156.704653 49.296205) (xy 158.202604 49.104555) (xy 159.708746 48.965926) (xy 161.222324 48.881719)
   (xy 162.742587 48.853338))
  (stroke (width 0.5) (type solid)) (fill no) (layer "Edge.Cuts"))
 (segment (start 140.6525 59.21375) (end 133.50875 66.3575) (width 0.2) (layer "F.Cu") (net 3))
 (segment (start 140.024 112.699) (end 122.3065 94.9815) (width 0.2) (layer "F.Cu") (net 3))
 (segment (start 133.50875 66.3575) (end 133.50875 83.02625) (width 0.2) (layer "F.Cu") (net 3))
 (segment (start 122.3065 94.9815) (end 122.3065 71.768436) (width 0.2) (layer "F.Cu") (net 3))
 (segment (start 149.0955 117.8955) (end 149.0955 125.00675) (width 0.2) (layer "F.Cu") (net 3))
 (segment (start 140.125 122.31875) (end 139.222 121.41575) (width 0.2) (layer "F.Cu") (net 3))
 (segment (start 139.222 113.501) (end 140.024 112.699) (width 0.2) (layer "F.Cu") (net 3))
 (segment (start 122.3065 71.768436) (end 127.717436 66.3575) (width 0.2) (layer "F.Cu") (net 3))
 (segment (start 152.67 78.26375) (end 162.08375 78.26375) (width 0.2) (layer "F.Cu") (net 3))
 (segment (start 152.55875 59.21375) (end 140.6525 59.21375) (width 0.2) (layer "F.Cu") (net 3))
 (segment (start 139.222 121.41575) (end 139.222 113.501) (width 0.2) (layer "F.Cu") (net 3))
 (segment (start 144.625 113.425) (end 149.0955 117.8955) (width 0.2) (layer "F.Cu") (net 3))
 (segment (start 143.899 112.699) (end 144.625 113.425) (width 0.2) (layer "F.Cu") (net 3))
 (segment (start 149.0955 125.00675) (end 150.6125 126.52375) (width 0.2) (layer "F.Cu") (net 3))
 (segment (start 133.50875 83.02625) (end 131.1275 85.4075) (width 0.2) (layer "F.Cu") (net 3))
 (segment (start 152.55875 78.1525) (end 147.685 83.02625) (width 0.2) (layer "F.Cu") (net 3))
 (segment (start 141.125 122.31875) (end 140.125 122.31875) (width 0.2) (layer "F.Cu") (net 3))
 (segment (start 127.717436 66.3575) (end 133.50875 66.3575) (width 0.2) (layer "F.Cu") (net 3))
 (segment (start 152.55875 59.21375) (end 152.55875 78.1525) (width 0.2) (layer "F.Cu") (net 3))
 (segment (start 152.55875 59.21375) (end 171.60875 59.21375) (width 0.2) (layer "F.Cu") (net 3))
 (segment (start 152.55875 78.1525) (end 152.67 78.26375) (width 0.2) (layer "F.Cu") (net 3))
 (segment (start 140.024 112.699) (end 143.899 112.699) (width 0.2) (layer "F.Cu") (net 3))
 (segment (start 127.15875 85.17975) (end 132.4665 90.4875) (width 0.2) (layer "F.Cu") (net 15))
 (segment (start 132.4665 94.84275) (end 151.4475 113.82375) (width 0.2) (layer "F.Cu") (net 15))
 (segment (start 132.4665 90.4875) (end 132.4665 94.84275) (width 0.2) (layer "F.Cu") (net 15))
 (segment (start 127.15875 68.8975) (end 127.15875 85.17975) (width 0.2) (layer "F.Cu") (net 15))
 (segment (start 124.7775 90.307376) (end 150.833874 116.36375) (width 0.2) (layer "F.Cu") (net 12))
 (segment (start 150.833874 116.36375) (end 151.4475 116.36375) (width 0.2) (layer "F.Cu") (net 12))
 (segment (start 124.7775 87.9475) (end 124.7775 90.307376) (width 0.2) (layer "F.Cu") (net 12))
 (segment (start 146.20875 78.711186) (end 138.864 86.055936) (width 0.2) (layer "F.Cu") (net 11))
 (segment (start 152.5105 113.38344) (end 152.5105 117.84075) (width 0.2) (layer "F.Cu") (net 11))
 (segment (start 138.864 99.73694) (end 152.5105 113.38344) (width 0.2) (layer "F.Cu") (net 11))
 (segment (start 146.20875 61.75375) (end 146.20875 78.711186) (width 0.2) (layer "F.Cu") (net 11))
 (segment (start 138.864 86.055936) (end 138.864 99.73694) (width 0.2) (layer "F.Cu") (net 11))
 (segment (start 152.5105 117.84075) (end 151.4475 118.90375) (width 0.2) (layer "F.Cu") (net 11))
 (segment (start 165.25875 61.75375) (end 166.6875 63.1825) (width 0.2) (layer "F.Cu") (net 5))
 (segment (start 166.6875 63.1825) (end 166.6875 113.82375) (width 0.2) (layer "F.Cu") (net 5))
 (segment (start 155.73375 80.80375) (end 155.73375 105.41) (width 0.2) (layer "F.Cu") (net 14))
 (segment (start 155.73375 105.41) (end 166.6875 116.36375) (width 0.2) (layer "F.Cu") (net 14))
 (segment (start 191.651 105.926) (end 190.5 104.775) (width 0.2) (layer "F.Cu") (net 9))
 (segment (start 183.35625 117.0625) (end 176.762376 117.0625) (width 0.2) (layer "F.Cu") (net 9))
 (segment (start 176.762376 117.0625) (end 168.364126 125.46075) (width 0.2) (layer "F.Cu") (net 9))
 (segment (start 191.651 110.76775) (end 191.651 105.926) (width 0.2) (layer "F.Cu") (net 9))
 (segment (start 190.5 111.91875) (end 191.651 110.76775) (width 0.2) (layer "F.Cu") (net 9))
 (segment (start 185.35625 117.0625) (end 183.35625 117.0625) (width 0.2) (layer "F.Cu") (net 9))
 (segment (start 190.5 111.91875) (end 185.35625 117.0625) (width 0.2) (layer "F.Cu") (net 9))
 (segment (start 152.9245 125.46075) (end 151.4475 123.98375) (width 0.2) (layer "F.Cu") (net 9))
 (segment (start 168.364126 125.46075) (end 152.9245 125.46075) (width 0.2) (layer "F.Cu") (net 9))
 (segment (start 188.95 108.865) (end 188.95 111.91875) (width 0.2) (layer "F.Cu") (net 4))
 (segment (start 190.5 107.315) (end 188.95 108.865) (width 0.2) (layer "F.Cu") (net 4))
 (segment (start 183.35625 121.0625) (end 182.29375 121.0625) (width 0.2) (layer "F.Cu") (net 4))
 (segment (start 182.29375 121.0625) (end 179.53125 123.825) (width 0.2) (layer "F.Cu") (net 4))
 (segment (start 174.65625 125.875) (end 174.65625 128.5875) (width 0.2) (layer "F.Cu") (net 2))
 (segment (start 177.65625 122.875) (end 174.65625 125.875) (width 0.2) (layer "F.Cu") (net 2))
 (segment (start 167.16375 128.5875) (end 166.6875 129.06375) (width 0.2) (layer "F.Cu") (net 1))
 (segment (start 173.00625 128.5875) (end 167.16375 128.5875) (width 0.2) (layer "F.Cu") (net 1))
 (segment (start 141.335 85.56625) (end 141.335 98.63125) (width 0.2) (layer "F.Cu") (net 10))
 (segment (start 141.335 98.63125) (end 166.6875 123.98375) (width 0.2) (layer "F.Cu") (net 10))
 (segment (start 140.024 117.71775) (end 144.625 122.31875) (width 0.2) (layer "F.Cu") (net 7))
 (segment (start 143.899 114.449) (end 140.024 114.449) (width 0.2) (layer "F.Cu") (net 7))
 (segment (start 140.024 114.449) (end 140.024 117.71775) (width 0.2) (layer "F.Cu") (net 7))
 (segment (start 144.625 115.175) (end 143.899 114.449) (width 0.2) (layer "F.Cu") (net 7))
 (segment (start 147.6375 126.33138) (end 150.36987 129.06375) (width 0.2) (layer "F.Cu") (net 8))
 (segment (start 144.625 120.56875) (end 144.625 118.675) (width 0.2) (layer "F.Cu") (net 8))
 (segment (start 150.36987 129.06375) (end 151.4475 129.06375) (width 0.2) (layer "F.Cu") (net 8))
 (segment (start 144.625 118.675) (end 141.125 115.175) (width 0.2) (layer "F.Cu") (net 8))
 (segment (start 144.625 120.56875) (end 147.6375 123.58125) (width 0.2) (layer "F.Cu") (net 8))
 (segment (start 147.6375 123.58125) (end 147.6375 126.33138) (width 0.2) (layer "F.Cu") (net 8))
 (segment (start 149.356874 130.12675) (end 163.0845 130.12675) (width 0.2) (layer "F.Cu") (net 13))
 (segment (start 139.623 114.2829) (end 139.623 120.89375) (width 0.2) (layer "F.Cu") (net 13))
 (segment (start 139.623 120.89375) (end 140.024 121.29475) (width 0.2) (layer "F.Cu") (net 13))
 (segment (start 142.226 121.29475) (end 142.226 122.995876) (width 0.2) (layer "F.Cu") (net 13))
 (segment (start 141.125 113.425) (end 140.4809 113.425) (width 0.2) (layer "F.Cu") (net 13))
 (segment (start 140.024 121.29475) (end 142.226 121.29475) (width 0.2) (layer "F.Cu") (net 13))
 (segment (start 163.0845 130.12675) (end 166.6875 126.52375) (width 0.2) (layer "F.Cu") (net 13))
 (segment (start 142.226 122.995876) (end 149.356874 130.12675) (width 0.2) (layer "F.Cu") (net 13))
 (segment (start 140.4809 113.425) (end 139.623 114.2829) (width 0.2) (layer "F.Cu") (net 13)))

